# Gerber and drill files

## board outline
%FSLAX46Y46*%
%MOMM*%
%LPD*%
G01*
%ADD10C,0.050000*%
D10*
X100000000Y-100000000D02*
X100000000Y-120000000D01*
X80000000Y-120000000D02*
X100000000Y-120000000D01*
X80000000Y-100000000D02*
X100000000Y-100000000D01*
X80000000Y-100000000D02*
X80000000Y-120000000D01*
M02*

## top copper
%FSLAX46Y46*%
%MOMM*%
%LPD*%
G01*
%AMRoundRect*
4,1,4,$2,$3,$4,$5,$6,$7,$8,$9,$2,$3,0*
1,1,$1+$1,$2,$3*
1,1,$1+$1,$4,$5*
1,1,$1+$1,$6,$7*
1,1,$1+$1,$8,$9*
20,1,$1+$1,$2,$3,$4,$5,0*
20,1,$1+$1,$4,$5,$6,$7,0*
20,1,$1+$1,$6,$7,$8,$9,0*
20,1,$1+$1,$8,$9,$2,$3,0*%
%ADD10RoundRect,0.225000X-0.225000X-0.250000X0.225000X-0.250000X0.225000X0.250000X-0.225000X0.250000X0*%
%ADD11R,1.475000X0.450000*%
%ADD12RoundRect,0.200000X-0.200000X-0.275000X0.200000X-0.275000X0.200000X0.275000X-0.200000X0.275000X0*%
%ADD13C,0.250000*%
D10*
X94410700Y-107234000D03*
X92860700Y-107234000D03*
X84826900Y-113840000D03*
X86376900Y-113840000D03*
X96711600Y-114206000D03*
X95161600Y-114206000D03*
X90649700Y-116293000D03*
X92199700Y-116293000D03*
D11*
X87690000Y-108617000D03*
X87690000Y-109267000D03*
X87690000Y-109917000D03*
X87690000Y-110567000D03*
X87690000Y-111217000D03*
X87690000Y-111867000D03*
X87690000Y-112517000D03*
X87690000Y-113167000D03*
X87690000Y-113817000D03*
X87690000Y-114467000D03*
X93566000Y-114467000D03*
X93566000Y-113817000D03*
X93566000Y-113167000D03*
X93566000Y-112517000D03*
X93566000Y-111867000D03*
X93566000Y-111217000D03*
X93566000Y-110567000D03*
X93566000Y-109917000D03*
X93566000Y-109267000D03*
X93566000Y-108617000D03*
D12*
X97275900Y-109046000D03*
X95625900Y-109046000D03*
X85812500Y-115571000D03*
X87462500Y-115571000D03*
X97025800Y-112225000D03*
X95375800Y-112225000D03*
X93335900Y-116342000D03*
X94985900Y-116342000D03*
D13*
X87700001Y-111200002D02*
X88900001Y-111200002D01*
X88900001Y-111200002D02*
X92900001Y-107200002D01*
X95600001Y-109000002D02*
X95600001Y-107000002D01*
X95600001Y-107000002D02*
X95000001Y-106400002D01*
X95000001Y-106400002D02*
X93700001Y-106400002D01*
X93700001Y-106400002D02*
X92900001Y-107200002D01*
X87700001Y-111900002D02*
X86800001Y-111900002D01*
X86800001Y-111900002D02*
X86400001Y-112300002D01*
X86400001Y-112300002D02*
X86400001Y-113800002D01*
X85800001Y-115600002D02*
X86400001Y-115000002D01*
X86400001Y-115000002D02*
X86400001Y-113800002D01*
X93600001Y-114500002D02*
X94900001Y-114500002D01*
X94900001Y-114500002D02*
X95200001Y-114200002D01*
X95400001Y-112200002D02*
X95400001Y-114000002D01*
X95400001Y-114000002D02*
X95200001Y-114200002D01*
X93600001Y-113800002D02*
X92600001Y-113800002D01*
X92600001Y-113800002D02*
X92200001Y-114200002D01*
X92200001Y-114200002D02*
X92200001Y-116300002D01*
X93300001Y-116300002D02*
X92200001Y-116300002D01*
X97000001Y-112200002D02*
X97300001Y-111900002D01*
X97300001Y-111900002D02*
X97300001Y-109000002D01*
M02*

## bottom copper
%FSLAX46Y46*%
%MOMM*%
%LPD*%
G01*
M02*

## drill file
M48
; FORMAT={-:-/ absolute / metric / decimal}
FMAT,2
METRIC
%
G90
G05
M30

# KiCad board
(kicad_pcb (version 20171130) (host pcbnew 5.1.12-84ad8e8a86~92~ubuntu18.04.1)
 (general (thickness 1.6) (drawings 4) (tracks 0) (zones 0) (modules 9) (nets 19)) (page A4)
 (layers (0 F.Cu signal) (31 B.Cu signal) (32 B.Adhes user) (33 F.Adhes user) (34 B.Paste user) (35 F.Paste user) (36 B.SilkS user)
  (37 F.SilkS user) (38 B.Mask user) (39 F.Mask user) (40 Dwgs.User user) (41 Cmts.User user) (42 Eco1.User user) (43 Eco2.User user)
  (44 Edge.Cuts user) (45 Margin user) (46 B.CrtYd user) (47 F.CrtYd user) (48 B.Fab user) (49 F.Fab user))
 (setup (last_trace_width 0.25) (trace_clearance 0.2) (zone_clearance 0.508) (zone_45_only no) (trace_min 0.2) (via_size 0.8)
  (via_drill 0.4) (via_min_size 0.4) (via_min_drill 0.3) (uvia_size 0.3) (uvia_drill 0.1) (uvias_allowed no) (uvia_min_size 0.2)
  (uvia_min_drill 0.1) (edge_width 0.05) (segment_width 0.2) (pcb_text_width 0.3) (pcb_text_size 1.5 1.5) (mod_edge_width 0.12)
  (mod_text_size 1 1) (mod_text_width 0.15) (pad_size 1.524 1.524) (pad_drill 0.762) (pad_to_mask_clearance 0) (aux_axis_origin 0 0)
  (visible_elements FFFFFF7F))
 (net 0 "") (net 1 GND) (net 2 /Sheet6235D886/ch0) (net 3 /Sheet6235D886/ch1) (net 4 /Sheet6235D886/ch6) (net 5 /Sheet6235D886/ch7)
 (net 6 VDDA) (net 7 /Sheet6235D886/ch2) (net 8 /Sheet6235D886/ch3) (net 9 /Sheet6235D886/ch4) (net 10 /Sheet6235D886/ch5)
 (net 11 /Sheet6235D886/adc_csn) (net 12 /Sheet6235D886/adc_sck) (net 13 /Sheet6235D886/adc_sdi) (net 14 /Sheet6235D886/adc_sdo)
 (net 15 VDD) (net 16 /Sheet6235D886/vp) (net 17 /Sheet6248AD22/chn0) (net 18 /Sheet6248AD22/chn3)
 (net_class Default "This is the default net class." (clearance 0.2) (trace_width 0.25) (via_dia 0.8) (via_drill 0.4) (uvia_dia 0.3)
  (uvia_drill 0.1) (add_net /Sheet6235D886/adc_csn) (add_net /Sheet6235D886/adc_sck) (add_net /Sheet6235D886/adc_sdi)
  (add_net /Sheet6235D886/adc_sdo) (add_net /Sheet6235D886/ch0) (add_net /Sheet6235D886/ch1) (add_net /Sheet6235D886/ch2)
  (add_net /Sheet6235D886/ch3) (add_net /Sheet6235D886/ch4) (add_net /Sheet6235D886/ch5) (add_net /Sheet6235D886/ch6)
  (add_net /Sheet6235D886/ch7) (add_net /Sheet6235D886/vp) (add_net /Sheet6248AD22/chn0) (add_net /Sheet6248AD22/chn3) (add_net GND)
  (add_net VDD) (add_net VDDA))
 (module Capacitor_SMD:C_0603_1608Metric (layer F.Cu) (at 93.635700 107.234000)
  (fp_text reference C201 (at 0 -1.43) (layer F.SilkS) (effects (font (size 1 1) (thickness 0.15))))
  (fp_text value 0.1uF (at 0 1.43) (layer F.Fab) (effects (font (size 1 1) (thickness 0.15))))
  (pad 2 smd roundrect (at 0.775 0) (size 0.9 0.95) (layers F.Cu F.Mask F.Paste) (roundrect_rratio 0.25) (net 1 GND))
  (pad 1 smd roundrect (at -0.775 0) (size 0.9 0.95) (layers F.Cu F.Mask F.Paste) (roundrect_rratio 0.25) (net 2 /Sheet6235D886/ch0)))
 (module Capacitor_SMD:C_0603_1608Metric (layer F.Cu) (at 85.601900 113.840000)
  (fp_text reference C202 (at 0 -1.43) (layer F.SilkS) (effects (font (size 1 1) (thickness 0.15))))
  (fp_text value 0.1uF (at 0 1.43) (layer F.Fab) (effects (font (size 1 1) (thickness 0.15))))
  (pad 1 smd roundrect (at -0.775 0) (size 0.9 0.95) (layers F.Cu F.Mask F.Paste) (roundrect_rratio 0.25) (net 1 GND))
  (pad 2 smd roundrect (at 0.775 0) (size 0.9 0.95) (layers F.Cu F.Mask F.Paste) (roundrect_rratio 0.25) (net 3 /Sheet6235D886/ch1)))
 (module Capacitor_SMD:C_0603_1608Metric (layer F.Cu) (at 95.936600 114.206000)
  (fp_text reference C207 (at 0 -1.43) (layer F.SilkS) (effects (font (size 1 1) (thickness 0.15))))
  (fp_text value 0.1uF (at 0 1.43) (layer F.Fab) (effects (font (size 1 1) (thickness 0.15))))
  (pad 2 smd roundrect (at 0.775 0) (size 0.9 0.95) (layers F.Cu F.Mask F.Paste) (roundrect_rratio 0.25) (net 1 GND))
  (pad 1 smd roundrect (at -0.775 0) (size 0.9 0.95) (layers F.Cu F.Mask F.Paste) (roundrect_rratio 0.25) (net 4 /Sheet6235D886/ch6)))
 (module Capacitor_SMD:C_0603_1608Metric (layer F.Cu) (at 91.424700 116.293000)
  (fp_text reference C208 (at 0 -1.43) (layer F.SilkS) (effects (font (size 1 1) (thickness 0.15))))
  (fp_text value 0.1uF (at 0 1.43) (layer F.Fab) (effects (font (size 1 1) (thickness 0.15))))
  (pad 1 smd roundrect (at -0.775 0) (size 0.9 0.95) (layers F.Cu F.Mask F.Paste) (roundrect_rratio 0.25) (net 1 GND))
  (pad 2 smd roundrect (at 0.775 0) (size 0.9 0.95) (layers F.Cu F.Mask F.Paste) (roundrect_rratio 0.25) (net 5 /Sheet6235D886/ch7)))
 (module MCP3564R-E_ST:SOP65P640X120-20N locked (layer F.Cu) (at 90.628000 111.542000)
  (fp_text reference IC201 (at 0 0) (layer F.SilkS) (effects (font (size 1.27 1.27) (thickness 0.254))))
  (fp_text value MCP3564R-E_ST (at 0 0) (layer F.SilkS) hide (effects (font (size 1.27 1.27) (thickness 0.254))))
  (pad 1 smd rect (at -2.938 -2.925 90.000000) (size 0.45 1.475) (layers F.Cu F.Mask F.Paste) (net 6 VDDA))
  (pad 2 smd rect (at -2.938 -2.275 90.000000) (size 0.45 1.475) (layers F.Cu F.Mask F.Paste) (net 1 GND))
  (pad 3 smd rect (at -2.938 -1.625 90.000000) (size 0.45 1.475) (layers F.Cu F.Mask F.Paste) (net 1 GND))
  (pad 4 smd rect (at -2.938 -0.975 90.000000) (size 0.45 1.475) (layers F.Cu F.Mask F.Paste))
  (pad 5 smd rect (at -2.938 -0.325 90.000000) (size 0.45 1.475) (layers F.Cu F.Mask F.Paste) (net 2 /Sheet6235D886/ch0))
  (pad 6 smd rect (at -2.938 0.325 90.000000) (size 0.45 1.475) (layers F.Cu F.Mask F.Paste) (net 3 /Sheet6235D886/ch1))
  (pad 7 smd rect (at -2.938 0.975 90.000000) (size 0.45 1.475) (layers F.Cu F.Mask F.Paste) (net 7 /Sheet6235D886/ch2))
  (pad 8 smd rect (at -2.938 1.625 90.000000) (size 0.45 1.475) (layers F.Cu F.Mask F.Paste) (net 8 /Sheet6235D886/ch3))
  (pad 9 smd rect (at -2.938 2.275 90.000000) (size 0.45 1.475) (layers F.Cu F.Mask F.Paste) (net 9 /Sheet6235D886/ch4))
  (pad 10 smd rect (at -2.938 2.925 90.000000) (size 0.45 1.475) (layers F.Cu F.Mask F.Paste) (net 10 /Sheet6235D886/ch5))
  (pad 11 smd rect (at 2.938 2.925 90.000000) (size 0.45 1.475) (layers F.Cu F.Mask F.Paste) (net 4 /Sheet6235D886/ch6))
  (pad 12 smd rect (at 2.938 2.275 90.000000) (size 0.45 1.475) (layers F.Cu F.Mask F.Paste) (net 5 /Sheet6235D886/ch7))
  (pad 13 smd rect (at 2.938 1.625 90.000000) (size 0.45 1.475) (layers F.Cu F.Mask F.Paste) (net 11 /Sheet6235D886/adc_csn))
  (pad 14 smd rect (at 2.938 0.975 90.000000) (size 0.45 1.475) (layers F.Cu F.Mask F.Paste) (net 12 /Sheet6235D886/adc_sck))
  (pad 15 smd rect (at 2.938 0.325 90.000000) (size 0.45 1.475) (layers F.Cu F.Mask F.Paste) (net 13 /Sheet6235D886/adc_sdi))
  (pad 16 smd rect (at 2.938 -0.325 90.000000) (size 0.45 1.475) (layers F.Cu F.Mask F.Paste) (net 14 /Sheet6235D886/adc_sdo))
  (pad 17 smd rect (at 2.938 -0.975 90.000000) (size 0.45 1.475) (layers F.Cu F.Mask F.Paste))
  (pad 18 smd rect (at 2.938 -1.625 90.000000) (size 0.45 1.475) (layers F.Cu F.Mask F.Paste))
  (pad 19 smd rect (at 2.938 -2.275 90.000000) (size 0.45 1.475) (layers F.Cu F.Mask F.Paste) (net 1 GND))
  (pad 20 smd rect (at 2.938 -2.925 90.000000) (size 0.45 1.475) (layers F.Cu F.Mask F.Paste) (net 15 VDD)))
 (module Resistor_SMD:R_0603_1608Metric (layer F.Cu) (at 96.450900 109.046000)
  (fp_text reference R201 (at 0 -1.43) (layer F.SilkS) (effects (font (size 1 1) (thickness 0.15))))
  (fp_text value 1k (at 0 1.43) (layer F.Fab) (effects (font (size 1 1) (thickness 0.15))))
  (pad 2 smd roundrect (at 0.825 0) (size 0.8 0.95) (layers F.Cu F.Mask F.Paste) (roundrect_rratio 0.25) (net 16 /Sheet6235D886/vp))
  (pad 1 smd roundrect (at -0.825 0) (size 0.8 0.95) (layers F.Cu F.Mask F.Paste) (roundrect_rratio 0.25) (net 2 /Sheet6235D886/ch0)))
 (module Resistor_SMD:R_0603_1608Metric (layer F.Cu) (at 86.637500 115.571000)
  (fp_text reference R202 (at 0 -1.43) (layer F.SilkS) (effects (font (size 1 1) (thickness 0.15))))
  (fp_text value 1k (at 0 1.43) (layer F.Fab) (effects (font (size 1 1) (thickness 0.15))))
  (pad 1 smd roundrect (at -0.825 0) (size 0.8 0.95) (layers F.Cu F.Mask F.Paste) (roundrect_rratio 0.25) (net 3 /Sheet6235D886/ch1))
  (pad 2 smd roundrect (at 0.825 0) (size 0.8 0.95) (layers F.Cu F.Mask F.Paste) (roundrect_rratio 0.25) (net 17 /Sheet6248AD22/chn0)))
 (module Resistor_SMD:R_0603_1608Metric (layer F.Cu) (at 96.200800 112.225000)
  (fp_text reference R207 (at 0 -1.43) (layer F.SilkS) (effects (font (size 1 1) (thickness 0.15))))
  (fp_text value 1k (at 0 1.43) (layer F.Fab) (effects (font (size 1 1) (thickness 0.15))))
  (pad 2 smd roundrect (at 0.825 0) (size 0.8 0.95) (layers F.Cu F.Mask F.Paste) (roundrect_rratio 0.25) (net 16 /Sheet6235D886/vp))
  (pad 1 smd roundrect (at -0.825 0) (size 0.8 0.95) (layers F.Cu F.Mask F.Paste) (roundrect_rratio 0.25) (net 4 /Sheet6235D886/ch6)))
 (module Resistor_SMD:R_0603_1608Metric (layer F.Cu) (at 94.160900 116.342000)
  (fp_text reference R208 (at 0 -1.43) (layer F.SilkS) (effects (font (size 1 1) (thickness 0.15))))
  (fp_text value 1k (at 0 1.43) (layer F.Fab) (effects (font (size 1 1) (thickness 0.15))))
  (pad 1 smd roundrect (at -0.825 0) (size 0.8 0.95) (layers F.Cu F.Mask F.Paste) (roundrect_rratio 0.25) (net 5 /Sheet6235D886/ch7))
  (pad 2 smd roundrect (at 0.825 0) (size 0.8 0.95) (layers F.Cu F.Mask F.Paste) (roundrect_rratio 0.25) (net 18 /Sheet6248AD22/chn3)))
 (gr_line (start 100 100) (end 100 120) (layer Edge.Cuts) (width 0.05))
 (gr_line (start 80 120) (end 100 120) (layer Edge.Cuts) (width 0.05))
 (gr_line (start 80 100) (end 100 100) (layer Edge.Cuts) (width 0.05))
 (gr_line (start 80 100) (end 80 120) (layer Edge.Cuts) (width 0.05))
 (segment (start 87.700001 111.200002) (end 88.900001 111.200002) (width 0.250000) (layer F.Cu) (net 2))
 (segment (start 88.900001 111.200002) (end 92.900001 107.200002) (width 0.250000) (layer F.Cu) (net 2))
 (segment (start 95.600001 109.000002) (end 95.600001 107.000002) (width 0.250000) (layer F.Cu) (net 2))
 (segment (start 95.600001 107.000002) (end 95.000001 106.400002) (width 0.250000) (layer F.Cu) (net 2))
 (segment (start 95.000001 106.400002) (end 93.700001 106.400002) (width 0.250000) (layer F.Cu) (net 2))
 (segment (start 93.700001 106.400002) (end 92.900001 107.200002) (width 0.250000) (layer F.Cu) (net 2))
 (segment (start 87.700001 111.900002) (end 86.800001 111.900002) (width 0.250000) (layer F.Cu) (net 3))
 (segment (start 86.800001 111.900002) (end 86.400001 112.300002) (width 0.250000) (layer F.Cu) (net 3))
 (segment (start 86.400001 112.300002) (end 86.400001 113.800002) (width 0.250000) (layer F.Cu) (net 3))
 (segment (start 85.800001 115.600002) (end 86.400001 115.000002) (width 0.250000) (layer F.Cu) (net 3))
 (segment (start 86.400001 115.000002) (end 86.400001 113.800002) (width 0.250000) (layer F.Cu) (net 3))
 (segment (start 93.600001 114.500002) (end 94.900001 114.500002) (width 0.250000) (layer F.Cu) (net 4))
 (segment (start 94.900001 114.500002) (end 95.200001 114.200002) (width 0.250000) (layer F.Cu) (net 4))
 (segment (start 95.400001 112.200002) (end 95.400001 114.000002) (width 0.250000) (layer F.Cu) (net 4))
 (segment (start 95.400001 114.000002) (end 95.200001 114.200002) (width 0.250000) (layer F.Cu) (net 4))
 (segment (start 93.600001 113.800002) (end 92.600001 113.800002) (width 0.250000) (layer F.Cu) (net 5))
 (segment (start 92.600001 113.800002) (end 92.200001 114.200002) (width 0.250000) (layer F.Cu) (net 5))
 (segment (start 92.200001 114.200002) (end 92.200001 116.300002) (width 0.250000) (layer F.Cu) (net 5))
 (segment (start 93.300001 116.300002) (end 92.200001 116.300002) (width 0.250000) (layer F.Cu) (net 5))
 (segment (start 97.000001 112.200002) (end 97.300001 111.900002) (width 0.250000) (layer F.Cu) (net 16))
 (segment (start 97.300001 111.900002) (end 97.300001 109.000002) (width 0.250000) (layer F.Cu) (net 16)))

